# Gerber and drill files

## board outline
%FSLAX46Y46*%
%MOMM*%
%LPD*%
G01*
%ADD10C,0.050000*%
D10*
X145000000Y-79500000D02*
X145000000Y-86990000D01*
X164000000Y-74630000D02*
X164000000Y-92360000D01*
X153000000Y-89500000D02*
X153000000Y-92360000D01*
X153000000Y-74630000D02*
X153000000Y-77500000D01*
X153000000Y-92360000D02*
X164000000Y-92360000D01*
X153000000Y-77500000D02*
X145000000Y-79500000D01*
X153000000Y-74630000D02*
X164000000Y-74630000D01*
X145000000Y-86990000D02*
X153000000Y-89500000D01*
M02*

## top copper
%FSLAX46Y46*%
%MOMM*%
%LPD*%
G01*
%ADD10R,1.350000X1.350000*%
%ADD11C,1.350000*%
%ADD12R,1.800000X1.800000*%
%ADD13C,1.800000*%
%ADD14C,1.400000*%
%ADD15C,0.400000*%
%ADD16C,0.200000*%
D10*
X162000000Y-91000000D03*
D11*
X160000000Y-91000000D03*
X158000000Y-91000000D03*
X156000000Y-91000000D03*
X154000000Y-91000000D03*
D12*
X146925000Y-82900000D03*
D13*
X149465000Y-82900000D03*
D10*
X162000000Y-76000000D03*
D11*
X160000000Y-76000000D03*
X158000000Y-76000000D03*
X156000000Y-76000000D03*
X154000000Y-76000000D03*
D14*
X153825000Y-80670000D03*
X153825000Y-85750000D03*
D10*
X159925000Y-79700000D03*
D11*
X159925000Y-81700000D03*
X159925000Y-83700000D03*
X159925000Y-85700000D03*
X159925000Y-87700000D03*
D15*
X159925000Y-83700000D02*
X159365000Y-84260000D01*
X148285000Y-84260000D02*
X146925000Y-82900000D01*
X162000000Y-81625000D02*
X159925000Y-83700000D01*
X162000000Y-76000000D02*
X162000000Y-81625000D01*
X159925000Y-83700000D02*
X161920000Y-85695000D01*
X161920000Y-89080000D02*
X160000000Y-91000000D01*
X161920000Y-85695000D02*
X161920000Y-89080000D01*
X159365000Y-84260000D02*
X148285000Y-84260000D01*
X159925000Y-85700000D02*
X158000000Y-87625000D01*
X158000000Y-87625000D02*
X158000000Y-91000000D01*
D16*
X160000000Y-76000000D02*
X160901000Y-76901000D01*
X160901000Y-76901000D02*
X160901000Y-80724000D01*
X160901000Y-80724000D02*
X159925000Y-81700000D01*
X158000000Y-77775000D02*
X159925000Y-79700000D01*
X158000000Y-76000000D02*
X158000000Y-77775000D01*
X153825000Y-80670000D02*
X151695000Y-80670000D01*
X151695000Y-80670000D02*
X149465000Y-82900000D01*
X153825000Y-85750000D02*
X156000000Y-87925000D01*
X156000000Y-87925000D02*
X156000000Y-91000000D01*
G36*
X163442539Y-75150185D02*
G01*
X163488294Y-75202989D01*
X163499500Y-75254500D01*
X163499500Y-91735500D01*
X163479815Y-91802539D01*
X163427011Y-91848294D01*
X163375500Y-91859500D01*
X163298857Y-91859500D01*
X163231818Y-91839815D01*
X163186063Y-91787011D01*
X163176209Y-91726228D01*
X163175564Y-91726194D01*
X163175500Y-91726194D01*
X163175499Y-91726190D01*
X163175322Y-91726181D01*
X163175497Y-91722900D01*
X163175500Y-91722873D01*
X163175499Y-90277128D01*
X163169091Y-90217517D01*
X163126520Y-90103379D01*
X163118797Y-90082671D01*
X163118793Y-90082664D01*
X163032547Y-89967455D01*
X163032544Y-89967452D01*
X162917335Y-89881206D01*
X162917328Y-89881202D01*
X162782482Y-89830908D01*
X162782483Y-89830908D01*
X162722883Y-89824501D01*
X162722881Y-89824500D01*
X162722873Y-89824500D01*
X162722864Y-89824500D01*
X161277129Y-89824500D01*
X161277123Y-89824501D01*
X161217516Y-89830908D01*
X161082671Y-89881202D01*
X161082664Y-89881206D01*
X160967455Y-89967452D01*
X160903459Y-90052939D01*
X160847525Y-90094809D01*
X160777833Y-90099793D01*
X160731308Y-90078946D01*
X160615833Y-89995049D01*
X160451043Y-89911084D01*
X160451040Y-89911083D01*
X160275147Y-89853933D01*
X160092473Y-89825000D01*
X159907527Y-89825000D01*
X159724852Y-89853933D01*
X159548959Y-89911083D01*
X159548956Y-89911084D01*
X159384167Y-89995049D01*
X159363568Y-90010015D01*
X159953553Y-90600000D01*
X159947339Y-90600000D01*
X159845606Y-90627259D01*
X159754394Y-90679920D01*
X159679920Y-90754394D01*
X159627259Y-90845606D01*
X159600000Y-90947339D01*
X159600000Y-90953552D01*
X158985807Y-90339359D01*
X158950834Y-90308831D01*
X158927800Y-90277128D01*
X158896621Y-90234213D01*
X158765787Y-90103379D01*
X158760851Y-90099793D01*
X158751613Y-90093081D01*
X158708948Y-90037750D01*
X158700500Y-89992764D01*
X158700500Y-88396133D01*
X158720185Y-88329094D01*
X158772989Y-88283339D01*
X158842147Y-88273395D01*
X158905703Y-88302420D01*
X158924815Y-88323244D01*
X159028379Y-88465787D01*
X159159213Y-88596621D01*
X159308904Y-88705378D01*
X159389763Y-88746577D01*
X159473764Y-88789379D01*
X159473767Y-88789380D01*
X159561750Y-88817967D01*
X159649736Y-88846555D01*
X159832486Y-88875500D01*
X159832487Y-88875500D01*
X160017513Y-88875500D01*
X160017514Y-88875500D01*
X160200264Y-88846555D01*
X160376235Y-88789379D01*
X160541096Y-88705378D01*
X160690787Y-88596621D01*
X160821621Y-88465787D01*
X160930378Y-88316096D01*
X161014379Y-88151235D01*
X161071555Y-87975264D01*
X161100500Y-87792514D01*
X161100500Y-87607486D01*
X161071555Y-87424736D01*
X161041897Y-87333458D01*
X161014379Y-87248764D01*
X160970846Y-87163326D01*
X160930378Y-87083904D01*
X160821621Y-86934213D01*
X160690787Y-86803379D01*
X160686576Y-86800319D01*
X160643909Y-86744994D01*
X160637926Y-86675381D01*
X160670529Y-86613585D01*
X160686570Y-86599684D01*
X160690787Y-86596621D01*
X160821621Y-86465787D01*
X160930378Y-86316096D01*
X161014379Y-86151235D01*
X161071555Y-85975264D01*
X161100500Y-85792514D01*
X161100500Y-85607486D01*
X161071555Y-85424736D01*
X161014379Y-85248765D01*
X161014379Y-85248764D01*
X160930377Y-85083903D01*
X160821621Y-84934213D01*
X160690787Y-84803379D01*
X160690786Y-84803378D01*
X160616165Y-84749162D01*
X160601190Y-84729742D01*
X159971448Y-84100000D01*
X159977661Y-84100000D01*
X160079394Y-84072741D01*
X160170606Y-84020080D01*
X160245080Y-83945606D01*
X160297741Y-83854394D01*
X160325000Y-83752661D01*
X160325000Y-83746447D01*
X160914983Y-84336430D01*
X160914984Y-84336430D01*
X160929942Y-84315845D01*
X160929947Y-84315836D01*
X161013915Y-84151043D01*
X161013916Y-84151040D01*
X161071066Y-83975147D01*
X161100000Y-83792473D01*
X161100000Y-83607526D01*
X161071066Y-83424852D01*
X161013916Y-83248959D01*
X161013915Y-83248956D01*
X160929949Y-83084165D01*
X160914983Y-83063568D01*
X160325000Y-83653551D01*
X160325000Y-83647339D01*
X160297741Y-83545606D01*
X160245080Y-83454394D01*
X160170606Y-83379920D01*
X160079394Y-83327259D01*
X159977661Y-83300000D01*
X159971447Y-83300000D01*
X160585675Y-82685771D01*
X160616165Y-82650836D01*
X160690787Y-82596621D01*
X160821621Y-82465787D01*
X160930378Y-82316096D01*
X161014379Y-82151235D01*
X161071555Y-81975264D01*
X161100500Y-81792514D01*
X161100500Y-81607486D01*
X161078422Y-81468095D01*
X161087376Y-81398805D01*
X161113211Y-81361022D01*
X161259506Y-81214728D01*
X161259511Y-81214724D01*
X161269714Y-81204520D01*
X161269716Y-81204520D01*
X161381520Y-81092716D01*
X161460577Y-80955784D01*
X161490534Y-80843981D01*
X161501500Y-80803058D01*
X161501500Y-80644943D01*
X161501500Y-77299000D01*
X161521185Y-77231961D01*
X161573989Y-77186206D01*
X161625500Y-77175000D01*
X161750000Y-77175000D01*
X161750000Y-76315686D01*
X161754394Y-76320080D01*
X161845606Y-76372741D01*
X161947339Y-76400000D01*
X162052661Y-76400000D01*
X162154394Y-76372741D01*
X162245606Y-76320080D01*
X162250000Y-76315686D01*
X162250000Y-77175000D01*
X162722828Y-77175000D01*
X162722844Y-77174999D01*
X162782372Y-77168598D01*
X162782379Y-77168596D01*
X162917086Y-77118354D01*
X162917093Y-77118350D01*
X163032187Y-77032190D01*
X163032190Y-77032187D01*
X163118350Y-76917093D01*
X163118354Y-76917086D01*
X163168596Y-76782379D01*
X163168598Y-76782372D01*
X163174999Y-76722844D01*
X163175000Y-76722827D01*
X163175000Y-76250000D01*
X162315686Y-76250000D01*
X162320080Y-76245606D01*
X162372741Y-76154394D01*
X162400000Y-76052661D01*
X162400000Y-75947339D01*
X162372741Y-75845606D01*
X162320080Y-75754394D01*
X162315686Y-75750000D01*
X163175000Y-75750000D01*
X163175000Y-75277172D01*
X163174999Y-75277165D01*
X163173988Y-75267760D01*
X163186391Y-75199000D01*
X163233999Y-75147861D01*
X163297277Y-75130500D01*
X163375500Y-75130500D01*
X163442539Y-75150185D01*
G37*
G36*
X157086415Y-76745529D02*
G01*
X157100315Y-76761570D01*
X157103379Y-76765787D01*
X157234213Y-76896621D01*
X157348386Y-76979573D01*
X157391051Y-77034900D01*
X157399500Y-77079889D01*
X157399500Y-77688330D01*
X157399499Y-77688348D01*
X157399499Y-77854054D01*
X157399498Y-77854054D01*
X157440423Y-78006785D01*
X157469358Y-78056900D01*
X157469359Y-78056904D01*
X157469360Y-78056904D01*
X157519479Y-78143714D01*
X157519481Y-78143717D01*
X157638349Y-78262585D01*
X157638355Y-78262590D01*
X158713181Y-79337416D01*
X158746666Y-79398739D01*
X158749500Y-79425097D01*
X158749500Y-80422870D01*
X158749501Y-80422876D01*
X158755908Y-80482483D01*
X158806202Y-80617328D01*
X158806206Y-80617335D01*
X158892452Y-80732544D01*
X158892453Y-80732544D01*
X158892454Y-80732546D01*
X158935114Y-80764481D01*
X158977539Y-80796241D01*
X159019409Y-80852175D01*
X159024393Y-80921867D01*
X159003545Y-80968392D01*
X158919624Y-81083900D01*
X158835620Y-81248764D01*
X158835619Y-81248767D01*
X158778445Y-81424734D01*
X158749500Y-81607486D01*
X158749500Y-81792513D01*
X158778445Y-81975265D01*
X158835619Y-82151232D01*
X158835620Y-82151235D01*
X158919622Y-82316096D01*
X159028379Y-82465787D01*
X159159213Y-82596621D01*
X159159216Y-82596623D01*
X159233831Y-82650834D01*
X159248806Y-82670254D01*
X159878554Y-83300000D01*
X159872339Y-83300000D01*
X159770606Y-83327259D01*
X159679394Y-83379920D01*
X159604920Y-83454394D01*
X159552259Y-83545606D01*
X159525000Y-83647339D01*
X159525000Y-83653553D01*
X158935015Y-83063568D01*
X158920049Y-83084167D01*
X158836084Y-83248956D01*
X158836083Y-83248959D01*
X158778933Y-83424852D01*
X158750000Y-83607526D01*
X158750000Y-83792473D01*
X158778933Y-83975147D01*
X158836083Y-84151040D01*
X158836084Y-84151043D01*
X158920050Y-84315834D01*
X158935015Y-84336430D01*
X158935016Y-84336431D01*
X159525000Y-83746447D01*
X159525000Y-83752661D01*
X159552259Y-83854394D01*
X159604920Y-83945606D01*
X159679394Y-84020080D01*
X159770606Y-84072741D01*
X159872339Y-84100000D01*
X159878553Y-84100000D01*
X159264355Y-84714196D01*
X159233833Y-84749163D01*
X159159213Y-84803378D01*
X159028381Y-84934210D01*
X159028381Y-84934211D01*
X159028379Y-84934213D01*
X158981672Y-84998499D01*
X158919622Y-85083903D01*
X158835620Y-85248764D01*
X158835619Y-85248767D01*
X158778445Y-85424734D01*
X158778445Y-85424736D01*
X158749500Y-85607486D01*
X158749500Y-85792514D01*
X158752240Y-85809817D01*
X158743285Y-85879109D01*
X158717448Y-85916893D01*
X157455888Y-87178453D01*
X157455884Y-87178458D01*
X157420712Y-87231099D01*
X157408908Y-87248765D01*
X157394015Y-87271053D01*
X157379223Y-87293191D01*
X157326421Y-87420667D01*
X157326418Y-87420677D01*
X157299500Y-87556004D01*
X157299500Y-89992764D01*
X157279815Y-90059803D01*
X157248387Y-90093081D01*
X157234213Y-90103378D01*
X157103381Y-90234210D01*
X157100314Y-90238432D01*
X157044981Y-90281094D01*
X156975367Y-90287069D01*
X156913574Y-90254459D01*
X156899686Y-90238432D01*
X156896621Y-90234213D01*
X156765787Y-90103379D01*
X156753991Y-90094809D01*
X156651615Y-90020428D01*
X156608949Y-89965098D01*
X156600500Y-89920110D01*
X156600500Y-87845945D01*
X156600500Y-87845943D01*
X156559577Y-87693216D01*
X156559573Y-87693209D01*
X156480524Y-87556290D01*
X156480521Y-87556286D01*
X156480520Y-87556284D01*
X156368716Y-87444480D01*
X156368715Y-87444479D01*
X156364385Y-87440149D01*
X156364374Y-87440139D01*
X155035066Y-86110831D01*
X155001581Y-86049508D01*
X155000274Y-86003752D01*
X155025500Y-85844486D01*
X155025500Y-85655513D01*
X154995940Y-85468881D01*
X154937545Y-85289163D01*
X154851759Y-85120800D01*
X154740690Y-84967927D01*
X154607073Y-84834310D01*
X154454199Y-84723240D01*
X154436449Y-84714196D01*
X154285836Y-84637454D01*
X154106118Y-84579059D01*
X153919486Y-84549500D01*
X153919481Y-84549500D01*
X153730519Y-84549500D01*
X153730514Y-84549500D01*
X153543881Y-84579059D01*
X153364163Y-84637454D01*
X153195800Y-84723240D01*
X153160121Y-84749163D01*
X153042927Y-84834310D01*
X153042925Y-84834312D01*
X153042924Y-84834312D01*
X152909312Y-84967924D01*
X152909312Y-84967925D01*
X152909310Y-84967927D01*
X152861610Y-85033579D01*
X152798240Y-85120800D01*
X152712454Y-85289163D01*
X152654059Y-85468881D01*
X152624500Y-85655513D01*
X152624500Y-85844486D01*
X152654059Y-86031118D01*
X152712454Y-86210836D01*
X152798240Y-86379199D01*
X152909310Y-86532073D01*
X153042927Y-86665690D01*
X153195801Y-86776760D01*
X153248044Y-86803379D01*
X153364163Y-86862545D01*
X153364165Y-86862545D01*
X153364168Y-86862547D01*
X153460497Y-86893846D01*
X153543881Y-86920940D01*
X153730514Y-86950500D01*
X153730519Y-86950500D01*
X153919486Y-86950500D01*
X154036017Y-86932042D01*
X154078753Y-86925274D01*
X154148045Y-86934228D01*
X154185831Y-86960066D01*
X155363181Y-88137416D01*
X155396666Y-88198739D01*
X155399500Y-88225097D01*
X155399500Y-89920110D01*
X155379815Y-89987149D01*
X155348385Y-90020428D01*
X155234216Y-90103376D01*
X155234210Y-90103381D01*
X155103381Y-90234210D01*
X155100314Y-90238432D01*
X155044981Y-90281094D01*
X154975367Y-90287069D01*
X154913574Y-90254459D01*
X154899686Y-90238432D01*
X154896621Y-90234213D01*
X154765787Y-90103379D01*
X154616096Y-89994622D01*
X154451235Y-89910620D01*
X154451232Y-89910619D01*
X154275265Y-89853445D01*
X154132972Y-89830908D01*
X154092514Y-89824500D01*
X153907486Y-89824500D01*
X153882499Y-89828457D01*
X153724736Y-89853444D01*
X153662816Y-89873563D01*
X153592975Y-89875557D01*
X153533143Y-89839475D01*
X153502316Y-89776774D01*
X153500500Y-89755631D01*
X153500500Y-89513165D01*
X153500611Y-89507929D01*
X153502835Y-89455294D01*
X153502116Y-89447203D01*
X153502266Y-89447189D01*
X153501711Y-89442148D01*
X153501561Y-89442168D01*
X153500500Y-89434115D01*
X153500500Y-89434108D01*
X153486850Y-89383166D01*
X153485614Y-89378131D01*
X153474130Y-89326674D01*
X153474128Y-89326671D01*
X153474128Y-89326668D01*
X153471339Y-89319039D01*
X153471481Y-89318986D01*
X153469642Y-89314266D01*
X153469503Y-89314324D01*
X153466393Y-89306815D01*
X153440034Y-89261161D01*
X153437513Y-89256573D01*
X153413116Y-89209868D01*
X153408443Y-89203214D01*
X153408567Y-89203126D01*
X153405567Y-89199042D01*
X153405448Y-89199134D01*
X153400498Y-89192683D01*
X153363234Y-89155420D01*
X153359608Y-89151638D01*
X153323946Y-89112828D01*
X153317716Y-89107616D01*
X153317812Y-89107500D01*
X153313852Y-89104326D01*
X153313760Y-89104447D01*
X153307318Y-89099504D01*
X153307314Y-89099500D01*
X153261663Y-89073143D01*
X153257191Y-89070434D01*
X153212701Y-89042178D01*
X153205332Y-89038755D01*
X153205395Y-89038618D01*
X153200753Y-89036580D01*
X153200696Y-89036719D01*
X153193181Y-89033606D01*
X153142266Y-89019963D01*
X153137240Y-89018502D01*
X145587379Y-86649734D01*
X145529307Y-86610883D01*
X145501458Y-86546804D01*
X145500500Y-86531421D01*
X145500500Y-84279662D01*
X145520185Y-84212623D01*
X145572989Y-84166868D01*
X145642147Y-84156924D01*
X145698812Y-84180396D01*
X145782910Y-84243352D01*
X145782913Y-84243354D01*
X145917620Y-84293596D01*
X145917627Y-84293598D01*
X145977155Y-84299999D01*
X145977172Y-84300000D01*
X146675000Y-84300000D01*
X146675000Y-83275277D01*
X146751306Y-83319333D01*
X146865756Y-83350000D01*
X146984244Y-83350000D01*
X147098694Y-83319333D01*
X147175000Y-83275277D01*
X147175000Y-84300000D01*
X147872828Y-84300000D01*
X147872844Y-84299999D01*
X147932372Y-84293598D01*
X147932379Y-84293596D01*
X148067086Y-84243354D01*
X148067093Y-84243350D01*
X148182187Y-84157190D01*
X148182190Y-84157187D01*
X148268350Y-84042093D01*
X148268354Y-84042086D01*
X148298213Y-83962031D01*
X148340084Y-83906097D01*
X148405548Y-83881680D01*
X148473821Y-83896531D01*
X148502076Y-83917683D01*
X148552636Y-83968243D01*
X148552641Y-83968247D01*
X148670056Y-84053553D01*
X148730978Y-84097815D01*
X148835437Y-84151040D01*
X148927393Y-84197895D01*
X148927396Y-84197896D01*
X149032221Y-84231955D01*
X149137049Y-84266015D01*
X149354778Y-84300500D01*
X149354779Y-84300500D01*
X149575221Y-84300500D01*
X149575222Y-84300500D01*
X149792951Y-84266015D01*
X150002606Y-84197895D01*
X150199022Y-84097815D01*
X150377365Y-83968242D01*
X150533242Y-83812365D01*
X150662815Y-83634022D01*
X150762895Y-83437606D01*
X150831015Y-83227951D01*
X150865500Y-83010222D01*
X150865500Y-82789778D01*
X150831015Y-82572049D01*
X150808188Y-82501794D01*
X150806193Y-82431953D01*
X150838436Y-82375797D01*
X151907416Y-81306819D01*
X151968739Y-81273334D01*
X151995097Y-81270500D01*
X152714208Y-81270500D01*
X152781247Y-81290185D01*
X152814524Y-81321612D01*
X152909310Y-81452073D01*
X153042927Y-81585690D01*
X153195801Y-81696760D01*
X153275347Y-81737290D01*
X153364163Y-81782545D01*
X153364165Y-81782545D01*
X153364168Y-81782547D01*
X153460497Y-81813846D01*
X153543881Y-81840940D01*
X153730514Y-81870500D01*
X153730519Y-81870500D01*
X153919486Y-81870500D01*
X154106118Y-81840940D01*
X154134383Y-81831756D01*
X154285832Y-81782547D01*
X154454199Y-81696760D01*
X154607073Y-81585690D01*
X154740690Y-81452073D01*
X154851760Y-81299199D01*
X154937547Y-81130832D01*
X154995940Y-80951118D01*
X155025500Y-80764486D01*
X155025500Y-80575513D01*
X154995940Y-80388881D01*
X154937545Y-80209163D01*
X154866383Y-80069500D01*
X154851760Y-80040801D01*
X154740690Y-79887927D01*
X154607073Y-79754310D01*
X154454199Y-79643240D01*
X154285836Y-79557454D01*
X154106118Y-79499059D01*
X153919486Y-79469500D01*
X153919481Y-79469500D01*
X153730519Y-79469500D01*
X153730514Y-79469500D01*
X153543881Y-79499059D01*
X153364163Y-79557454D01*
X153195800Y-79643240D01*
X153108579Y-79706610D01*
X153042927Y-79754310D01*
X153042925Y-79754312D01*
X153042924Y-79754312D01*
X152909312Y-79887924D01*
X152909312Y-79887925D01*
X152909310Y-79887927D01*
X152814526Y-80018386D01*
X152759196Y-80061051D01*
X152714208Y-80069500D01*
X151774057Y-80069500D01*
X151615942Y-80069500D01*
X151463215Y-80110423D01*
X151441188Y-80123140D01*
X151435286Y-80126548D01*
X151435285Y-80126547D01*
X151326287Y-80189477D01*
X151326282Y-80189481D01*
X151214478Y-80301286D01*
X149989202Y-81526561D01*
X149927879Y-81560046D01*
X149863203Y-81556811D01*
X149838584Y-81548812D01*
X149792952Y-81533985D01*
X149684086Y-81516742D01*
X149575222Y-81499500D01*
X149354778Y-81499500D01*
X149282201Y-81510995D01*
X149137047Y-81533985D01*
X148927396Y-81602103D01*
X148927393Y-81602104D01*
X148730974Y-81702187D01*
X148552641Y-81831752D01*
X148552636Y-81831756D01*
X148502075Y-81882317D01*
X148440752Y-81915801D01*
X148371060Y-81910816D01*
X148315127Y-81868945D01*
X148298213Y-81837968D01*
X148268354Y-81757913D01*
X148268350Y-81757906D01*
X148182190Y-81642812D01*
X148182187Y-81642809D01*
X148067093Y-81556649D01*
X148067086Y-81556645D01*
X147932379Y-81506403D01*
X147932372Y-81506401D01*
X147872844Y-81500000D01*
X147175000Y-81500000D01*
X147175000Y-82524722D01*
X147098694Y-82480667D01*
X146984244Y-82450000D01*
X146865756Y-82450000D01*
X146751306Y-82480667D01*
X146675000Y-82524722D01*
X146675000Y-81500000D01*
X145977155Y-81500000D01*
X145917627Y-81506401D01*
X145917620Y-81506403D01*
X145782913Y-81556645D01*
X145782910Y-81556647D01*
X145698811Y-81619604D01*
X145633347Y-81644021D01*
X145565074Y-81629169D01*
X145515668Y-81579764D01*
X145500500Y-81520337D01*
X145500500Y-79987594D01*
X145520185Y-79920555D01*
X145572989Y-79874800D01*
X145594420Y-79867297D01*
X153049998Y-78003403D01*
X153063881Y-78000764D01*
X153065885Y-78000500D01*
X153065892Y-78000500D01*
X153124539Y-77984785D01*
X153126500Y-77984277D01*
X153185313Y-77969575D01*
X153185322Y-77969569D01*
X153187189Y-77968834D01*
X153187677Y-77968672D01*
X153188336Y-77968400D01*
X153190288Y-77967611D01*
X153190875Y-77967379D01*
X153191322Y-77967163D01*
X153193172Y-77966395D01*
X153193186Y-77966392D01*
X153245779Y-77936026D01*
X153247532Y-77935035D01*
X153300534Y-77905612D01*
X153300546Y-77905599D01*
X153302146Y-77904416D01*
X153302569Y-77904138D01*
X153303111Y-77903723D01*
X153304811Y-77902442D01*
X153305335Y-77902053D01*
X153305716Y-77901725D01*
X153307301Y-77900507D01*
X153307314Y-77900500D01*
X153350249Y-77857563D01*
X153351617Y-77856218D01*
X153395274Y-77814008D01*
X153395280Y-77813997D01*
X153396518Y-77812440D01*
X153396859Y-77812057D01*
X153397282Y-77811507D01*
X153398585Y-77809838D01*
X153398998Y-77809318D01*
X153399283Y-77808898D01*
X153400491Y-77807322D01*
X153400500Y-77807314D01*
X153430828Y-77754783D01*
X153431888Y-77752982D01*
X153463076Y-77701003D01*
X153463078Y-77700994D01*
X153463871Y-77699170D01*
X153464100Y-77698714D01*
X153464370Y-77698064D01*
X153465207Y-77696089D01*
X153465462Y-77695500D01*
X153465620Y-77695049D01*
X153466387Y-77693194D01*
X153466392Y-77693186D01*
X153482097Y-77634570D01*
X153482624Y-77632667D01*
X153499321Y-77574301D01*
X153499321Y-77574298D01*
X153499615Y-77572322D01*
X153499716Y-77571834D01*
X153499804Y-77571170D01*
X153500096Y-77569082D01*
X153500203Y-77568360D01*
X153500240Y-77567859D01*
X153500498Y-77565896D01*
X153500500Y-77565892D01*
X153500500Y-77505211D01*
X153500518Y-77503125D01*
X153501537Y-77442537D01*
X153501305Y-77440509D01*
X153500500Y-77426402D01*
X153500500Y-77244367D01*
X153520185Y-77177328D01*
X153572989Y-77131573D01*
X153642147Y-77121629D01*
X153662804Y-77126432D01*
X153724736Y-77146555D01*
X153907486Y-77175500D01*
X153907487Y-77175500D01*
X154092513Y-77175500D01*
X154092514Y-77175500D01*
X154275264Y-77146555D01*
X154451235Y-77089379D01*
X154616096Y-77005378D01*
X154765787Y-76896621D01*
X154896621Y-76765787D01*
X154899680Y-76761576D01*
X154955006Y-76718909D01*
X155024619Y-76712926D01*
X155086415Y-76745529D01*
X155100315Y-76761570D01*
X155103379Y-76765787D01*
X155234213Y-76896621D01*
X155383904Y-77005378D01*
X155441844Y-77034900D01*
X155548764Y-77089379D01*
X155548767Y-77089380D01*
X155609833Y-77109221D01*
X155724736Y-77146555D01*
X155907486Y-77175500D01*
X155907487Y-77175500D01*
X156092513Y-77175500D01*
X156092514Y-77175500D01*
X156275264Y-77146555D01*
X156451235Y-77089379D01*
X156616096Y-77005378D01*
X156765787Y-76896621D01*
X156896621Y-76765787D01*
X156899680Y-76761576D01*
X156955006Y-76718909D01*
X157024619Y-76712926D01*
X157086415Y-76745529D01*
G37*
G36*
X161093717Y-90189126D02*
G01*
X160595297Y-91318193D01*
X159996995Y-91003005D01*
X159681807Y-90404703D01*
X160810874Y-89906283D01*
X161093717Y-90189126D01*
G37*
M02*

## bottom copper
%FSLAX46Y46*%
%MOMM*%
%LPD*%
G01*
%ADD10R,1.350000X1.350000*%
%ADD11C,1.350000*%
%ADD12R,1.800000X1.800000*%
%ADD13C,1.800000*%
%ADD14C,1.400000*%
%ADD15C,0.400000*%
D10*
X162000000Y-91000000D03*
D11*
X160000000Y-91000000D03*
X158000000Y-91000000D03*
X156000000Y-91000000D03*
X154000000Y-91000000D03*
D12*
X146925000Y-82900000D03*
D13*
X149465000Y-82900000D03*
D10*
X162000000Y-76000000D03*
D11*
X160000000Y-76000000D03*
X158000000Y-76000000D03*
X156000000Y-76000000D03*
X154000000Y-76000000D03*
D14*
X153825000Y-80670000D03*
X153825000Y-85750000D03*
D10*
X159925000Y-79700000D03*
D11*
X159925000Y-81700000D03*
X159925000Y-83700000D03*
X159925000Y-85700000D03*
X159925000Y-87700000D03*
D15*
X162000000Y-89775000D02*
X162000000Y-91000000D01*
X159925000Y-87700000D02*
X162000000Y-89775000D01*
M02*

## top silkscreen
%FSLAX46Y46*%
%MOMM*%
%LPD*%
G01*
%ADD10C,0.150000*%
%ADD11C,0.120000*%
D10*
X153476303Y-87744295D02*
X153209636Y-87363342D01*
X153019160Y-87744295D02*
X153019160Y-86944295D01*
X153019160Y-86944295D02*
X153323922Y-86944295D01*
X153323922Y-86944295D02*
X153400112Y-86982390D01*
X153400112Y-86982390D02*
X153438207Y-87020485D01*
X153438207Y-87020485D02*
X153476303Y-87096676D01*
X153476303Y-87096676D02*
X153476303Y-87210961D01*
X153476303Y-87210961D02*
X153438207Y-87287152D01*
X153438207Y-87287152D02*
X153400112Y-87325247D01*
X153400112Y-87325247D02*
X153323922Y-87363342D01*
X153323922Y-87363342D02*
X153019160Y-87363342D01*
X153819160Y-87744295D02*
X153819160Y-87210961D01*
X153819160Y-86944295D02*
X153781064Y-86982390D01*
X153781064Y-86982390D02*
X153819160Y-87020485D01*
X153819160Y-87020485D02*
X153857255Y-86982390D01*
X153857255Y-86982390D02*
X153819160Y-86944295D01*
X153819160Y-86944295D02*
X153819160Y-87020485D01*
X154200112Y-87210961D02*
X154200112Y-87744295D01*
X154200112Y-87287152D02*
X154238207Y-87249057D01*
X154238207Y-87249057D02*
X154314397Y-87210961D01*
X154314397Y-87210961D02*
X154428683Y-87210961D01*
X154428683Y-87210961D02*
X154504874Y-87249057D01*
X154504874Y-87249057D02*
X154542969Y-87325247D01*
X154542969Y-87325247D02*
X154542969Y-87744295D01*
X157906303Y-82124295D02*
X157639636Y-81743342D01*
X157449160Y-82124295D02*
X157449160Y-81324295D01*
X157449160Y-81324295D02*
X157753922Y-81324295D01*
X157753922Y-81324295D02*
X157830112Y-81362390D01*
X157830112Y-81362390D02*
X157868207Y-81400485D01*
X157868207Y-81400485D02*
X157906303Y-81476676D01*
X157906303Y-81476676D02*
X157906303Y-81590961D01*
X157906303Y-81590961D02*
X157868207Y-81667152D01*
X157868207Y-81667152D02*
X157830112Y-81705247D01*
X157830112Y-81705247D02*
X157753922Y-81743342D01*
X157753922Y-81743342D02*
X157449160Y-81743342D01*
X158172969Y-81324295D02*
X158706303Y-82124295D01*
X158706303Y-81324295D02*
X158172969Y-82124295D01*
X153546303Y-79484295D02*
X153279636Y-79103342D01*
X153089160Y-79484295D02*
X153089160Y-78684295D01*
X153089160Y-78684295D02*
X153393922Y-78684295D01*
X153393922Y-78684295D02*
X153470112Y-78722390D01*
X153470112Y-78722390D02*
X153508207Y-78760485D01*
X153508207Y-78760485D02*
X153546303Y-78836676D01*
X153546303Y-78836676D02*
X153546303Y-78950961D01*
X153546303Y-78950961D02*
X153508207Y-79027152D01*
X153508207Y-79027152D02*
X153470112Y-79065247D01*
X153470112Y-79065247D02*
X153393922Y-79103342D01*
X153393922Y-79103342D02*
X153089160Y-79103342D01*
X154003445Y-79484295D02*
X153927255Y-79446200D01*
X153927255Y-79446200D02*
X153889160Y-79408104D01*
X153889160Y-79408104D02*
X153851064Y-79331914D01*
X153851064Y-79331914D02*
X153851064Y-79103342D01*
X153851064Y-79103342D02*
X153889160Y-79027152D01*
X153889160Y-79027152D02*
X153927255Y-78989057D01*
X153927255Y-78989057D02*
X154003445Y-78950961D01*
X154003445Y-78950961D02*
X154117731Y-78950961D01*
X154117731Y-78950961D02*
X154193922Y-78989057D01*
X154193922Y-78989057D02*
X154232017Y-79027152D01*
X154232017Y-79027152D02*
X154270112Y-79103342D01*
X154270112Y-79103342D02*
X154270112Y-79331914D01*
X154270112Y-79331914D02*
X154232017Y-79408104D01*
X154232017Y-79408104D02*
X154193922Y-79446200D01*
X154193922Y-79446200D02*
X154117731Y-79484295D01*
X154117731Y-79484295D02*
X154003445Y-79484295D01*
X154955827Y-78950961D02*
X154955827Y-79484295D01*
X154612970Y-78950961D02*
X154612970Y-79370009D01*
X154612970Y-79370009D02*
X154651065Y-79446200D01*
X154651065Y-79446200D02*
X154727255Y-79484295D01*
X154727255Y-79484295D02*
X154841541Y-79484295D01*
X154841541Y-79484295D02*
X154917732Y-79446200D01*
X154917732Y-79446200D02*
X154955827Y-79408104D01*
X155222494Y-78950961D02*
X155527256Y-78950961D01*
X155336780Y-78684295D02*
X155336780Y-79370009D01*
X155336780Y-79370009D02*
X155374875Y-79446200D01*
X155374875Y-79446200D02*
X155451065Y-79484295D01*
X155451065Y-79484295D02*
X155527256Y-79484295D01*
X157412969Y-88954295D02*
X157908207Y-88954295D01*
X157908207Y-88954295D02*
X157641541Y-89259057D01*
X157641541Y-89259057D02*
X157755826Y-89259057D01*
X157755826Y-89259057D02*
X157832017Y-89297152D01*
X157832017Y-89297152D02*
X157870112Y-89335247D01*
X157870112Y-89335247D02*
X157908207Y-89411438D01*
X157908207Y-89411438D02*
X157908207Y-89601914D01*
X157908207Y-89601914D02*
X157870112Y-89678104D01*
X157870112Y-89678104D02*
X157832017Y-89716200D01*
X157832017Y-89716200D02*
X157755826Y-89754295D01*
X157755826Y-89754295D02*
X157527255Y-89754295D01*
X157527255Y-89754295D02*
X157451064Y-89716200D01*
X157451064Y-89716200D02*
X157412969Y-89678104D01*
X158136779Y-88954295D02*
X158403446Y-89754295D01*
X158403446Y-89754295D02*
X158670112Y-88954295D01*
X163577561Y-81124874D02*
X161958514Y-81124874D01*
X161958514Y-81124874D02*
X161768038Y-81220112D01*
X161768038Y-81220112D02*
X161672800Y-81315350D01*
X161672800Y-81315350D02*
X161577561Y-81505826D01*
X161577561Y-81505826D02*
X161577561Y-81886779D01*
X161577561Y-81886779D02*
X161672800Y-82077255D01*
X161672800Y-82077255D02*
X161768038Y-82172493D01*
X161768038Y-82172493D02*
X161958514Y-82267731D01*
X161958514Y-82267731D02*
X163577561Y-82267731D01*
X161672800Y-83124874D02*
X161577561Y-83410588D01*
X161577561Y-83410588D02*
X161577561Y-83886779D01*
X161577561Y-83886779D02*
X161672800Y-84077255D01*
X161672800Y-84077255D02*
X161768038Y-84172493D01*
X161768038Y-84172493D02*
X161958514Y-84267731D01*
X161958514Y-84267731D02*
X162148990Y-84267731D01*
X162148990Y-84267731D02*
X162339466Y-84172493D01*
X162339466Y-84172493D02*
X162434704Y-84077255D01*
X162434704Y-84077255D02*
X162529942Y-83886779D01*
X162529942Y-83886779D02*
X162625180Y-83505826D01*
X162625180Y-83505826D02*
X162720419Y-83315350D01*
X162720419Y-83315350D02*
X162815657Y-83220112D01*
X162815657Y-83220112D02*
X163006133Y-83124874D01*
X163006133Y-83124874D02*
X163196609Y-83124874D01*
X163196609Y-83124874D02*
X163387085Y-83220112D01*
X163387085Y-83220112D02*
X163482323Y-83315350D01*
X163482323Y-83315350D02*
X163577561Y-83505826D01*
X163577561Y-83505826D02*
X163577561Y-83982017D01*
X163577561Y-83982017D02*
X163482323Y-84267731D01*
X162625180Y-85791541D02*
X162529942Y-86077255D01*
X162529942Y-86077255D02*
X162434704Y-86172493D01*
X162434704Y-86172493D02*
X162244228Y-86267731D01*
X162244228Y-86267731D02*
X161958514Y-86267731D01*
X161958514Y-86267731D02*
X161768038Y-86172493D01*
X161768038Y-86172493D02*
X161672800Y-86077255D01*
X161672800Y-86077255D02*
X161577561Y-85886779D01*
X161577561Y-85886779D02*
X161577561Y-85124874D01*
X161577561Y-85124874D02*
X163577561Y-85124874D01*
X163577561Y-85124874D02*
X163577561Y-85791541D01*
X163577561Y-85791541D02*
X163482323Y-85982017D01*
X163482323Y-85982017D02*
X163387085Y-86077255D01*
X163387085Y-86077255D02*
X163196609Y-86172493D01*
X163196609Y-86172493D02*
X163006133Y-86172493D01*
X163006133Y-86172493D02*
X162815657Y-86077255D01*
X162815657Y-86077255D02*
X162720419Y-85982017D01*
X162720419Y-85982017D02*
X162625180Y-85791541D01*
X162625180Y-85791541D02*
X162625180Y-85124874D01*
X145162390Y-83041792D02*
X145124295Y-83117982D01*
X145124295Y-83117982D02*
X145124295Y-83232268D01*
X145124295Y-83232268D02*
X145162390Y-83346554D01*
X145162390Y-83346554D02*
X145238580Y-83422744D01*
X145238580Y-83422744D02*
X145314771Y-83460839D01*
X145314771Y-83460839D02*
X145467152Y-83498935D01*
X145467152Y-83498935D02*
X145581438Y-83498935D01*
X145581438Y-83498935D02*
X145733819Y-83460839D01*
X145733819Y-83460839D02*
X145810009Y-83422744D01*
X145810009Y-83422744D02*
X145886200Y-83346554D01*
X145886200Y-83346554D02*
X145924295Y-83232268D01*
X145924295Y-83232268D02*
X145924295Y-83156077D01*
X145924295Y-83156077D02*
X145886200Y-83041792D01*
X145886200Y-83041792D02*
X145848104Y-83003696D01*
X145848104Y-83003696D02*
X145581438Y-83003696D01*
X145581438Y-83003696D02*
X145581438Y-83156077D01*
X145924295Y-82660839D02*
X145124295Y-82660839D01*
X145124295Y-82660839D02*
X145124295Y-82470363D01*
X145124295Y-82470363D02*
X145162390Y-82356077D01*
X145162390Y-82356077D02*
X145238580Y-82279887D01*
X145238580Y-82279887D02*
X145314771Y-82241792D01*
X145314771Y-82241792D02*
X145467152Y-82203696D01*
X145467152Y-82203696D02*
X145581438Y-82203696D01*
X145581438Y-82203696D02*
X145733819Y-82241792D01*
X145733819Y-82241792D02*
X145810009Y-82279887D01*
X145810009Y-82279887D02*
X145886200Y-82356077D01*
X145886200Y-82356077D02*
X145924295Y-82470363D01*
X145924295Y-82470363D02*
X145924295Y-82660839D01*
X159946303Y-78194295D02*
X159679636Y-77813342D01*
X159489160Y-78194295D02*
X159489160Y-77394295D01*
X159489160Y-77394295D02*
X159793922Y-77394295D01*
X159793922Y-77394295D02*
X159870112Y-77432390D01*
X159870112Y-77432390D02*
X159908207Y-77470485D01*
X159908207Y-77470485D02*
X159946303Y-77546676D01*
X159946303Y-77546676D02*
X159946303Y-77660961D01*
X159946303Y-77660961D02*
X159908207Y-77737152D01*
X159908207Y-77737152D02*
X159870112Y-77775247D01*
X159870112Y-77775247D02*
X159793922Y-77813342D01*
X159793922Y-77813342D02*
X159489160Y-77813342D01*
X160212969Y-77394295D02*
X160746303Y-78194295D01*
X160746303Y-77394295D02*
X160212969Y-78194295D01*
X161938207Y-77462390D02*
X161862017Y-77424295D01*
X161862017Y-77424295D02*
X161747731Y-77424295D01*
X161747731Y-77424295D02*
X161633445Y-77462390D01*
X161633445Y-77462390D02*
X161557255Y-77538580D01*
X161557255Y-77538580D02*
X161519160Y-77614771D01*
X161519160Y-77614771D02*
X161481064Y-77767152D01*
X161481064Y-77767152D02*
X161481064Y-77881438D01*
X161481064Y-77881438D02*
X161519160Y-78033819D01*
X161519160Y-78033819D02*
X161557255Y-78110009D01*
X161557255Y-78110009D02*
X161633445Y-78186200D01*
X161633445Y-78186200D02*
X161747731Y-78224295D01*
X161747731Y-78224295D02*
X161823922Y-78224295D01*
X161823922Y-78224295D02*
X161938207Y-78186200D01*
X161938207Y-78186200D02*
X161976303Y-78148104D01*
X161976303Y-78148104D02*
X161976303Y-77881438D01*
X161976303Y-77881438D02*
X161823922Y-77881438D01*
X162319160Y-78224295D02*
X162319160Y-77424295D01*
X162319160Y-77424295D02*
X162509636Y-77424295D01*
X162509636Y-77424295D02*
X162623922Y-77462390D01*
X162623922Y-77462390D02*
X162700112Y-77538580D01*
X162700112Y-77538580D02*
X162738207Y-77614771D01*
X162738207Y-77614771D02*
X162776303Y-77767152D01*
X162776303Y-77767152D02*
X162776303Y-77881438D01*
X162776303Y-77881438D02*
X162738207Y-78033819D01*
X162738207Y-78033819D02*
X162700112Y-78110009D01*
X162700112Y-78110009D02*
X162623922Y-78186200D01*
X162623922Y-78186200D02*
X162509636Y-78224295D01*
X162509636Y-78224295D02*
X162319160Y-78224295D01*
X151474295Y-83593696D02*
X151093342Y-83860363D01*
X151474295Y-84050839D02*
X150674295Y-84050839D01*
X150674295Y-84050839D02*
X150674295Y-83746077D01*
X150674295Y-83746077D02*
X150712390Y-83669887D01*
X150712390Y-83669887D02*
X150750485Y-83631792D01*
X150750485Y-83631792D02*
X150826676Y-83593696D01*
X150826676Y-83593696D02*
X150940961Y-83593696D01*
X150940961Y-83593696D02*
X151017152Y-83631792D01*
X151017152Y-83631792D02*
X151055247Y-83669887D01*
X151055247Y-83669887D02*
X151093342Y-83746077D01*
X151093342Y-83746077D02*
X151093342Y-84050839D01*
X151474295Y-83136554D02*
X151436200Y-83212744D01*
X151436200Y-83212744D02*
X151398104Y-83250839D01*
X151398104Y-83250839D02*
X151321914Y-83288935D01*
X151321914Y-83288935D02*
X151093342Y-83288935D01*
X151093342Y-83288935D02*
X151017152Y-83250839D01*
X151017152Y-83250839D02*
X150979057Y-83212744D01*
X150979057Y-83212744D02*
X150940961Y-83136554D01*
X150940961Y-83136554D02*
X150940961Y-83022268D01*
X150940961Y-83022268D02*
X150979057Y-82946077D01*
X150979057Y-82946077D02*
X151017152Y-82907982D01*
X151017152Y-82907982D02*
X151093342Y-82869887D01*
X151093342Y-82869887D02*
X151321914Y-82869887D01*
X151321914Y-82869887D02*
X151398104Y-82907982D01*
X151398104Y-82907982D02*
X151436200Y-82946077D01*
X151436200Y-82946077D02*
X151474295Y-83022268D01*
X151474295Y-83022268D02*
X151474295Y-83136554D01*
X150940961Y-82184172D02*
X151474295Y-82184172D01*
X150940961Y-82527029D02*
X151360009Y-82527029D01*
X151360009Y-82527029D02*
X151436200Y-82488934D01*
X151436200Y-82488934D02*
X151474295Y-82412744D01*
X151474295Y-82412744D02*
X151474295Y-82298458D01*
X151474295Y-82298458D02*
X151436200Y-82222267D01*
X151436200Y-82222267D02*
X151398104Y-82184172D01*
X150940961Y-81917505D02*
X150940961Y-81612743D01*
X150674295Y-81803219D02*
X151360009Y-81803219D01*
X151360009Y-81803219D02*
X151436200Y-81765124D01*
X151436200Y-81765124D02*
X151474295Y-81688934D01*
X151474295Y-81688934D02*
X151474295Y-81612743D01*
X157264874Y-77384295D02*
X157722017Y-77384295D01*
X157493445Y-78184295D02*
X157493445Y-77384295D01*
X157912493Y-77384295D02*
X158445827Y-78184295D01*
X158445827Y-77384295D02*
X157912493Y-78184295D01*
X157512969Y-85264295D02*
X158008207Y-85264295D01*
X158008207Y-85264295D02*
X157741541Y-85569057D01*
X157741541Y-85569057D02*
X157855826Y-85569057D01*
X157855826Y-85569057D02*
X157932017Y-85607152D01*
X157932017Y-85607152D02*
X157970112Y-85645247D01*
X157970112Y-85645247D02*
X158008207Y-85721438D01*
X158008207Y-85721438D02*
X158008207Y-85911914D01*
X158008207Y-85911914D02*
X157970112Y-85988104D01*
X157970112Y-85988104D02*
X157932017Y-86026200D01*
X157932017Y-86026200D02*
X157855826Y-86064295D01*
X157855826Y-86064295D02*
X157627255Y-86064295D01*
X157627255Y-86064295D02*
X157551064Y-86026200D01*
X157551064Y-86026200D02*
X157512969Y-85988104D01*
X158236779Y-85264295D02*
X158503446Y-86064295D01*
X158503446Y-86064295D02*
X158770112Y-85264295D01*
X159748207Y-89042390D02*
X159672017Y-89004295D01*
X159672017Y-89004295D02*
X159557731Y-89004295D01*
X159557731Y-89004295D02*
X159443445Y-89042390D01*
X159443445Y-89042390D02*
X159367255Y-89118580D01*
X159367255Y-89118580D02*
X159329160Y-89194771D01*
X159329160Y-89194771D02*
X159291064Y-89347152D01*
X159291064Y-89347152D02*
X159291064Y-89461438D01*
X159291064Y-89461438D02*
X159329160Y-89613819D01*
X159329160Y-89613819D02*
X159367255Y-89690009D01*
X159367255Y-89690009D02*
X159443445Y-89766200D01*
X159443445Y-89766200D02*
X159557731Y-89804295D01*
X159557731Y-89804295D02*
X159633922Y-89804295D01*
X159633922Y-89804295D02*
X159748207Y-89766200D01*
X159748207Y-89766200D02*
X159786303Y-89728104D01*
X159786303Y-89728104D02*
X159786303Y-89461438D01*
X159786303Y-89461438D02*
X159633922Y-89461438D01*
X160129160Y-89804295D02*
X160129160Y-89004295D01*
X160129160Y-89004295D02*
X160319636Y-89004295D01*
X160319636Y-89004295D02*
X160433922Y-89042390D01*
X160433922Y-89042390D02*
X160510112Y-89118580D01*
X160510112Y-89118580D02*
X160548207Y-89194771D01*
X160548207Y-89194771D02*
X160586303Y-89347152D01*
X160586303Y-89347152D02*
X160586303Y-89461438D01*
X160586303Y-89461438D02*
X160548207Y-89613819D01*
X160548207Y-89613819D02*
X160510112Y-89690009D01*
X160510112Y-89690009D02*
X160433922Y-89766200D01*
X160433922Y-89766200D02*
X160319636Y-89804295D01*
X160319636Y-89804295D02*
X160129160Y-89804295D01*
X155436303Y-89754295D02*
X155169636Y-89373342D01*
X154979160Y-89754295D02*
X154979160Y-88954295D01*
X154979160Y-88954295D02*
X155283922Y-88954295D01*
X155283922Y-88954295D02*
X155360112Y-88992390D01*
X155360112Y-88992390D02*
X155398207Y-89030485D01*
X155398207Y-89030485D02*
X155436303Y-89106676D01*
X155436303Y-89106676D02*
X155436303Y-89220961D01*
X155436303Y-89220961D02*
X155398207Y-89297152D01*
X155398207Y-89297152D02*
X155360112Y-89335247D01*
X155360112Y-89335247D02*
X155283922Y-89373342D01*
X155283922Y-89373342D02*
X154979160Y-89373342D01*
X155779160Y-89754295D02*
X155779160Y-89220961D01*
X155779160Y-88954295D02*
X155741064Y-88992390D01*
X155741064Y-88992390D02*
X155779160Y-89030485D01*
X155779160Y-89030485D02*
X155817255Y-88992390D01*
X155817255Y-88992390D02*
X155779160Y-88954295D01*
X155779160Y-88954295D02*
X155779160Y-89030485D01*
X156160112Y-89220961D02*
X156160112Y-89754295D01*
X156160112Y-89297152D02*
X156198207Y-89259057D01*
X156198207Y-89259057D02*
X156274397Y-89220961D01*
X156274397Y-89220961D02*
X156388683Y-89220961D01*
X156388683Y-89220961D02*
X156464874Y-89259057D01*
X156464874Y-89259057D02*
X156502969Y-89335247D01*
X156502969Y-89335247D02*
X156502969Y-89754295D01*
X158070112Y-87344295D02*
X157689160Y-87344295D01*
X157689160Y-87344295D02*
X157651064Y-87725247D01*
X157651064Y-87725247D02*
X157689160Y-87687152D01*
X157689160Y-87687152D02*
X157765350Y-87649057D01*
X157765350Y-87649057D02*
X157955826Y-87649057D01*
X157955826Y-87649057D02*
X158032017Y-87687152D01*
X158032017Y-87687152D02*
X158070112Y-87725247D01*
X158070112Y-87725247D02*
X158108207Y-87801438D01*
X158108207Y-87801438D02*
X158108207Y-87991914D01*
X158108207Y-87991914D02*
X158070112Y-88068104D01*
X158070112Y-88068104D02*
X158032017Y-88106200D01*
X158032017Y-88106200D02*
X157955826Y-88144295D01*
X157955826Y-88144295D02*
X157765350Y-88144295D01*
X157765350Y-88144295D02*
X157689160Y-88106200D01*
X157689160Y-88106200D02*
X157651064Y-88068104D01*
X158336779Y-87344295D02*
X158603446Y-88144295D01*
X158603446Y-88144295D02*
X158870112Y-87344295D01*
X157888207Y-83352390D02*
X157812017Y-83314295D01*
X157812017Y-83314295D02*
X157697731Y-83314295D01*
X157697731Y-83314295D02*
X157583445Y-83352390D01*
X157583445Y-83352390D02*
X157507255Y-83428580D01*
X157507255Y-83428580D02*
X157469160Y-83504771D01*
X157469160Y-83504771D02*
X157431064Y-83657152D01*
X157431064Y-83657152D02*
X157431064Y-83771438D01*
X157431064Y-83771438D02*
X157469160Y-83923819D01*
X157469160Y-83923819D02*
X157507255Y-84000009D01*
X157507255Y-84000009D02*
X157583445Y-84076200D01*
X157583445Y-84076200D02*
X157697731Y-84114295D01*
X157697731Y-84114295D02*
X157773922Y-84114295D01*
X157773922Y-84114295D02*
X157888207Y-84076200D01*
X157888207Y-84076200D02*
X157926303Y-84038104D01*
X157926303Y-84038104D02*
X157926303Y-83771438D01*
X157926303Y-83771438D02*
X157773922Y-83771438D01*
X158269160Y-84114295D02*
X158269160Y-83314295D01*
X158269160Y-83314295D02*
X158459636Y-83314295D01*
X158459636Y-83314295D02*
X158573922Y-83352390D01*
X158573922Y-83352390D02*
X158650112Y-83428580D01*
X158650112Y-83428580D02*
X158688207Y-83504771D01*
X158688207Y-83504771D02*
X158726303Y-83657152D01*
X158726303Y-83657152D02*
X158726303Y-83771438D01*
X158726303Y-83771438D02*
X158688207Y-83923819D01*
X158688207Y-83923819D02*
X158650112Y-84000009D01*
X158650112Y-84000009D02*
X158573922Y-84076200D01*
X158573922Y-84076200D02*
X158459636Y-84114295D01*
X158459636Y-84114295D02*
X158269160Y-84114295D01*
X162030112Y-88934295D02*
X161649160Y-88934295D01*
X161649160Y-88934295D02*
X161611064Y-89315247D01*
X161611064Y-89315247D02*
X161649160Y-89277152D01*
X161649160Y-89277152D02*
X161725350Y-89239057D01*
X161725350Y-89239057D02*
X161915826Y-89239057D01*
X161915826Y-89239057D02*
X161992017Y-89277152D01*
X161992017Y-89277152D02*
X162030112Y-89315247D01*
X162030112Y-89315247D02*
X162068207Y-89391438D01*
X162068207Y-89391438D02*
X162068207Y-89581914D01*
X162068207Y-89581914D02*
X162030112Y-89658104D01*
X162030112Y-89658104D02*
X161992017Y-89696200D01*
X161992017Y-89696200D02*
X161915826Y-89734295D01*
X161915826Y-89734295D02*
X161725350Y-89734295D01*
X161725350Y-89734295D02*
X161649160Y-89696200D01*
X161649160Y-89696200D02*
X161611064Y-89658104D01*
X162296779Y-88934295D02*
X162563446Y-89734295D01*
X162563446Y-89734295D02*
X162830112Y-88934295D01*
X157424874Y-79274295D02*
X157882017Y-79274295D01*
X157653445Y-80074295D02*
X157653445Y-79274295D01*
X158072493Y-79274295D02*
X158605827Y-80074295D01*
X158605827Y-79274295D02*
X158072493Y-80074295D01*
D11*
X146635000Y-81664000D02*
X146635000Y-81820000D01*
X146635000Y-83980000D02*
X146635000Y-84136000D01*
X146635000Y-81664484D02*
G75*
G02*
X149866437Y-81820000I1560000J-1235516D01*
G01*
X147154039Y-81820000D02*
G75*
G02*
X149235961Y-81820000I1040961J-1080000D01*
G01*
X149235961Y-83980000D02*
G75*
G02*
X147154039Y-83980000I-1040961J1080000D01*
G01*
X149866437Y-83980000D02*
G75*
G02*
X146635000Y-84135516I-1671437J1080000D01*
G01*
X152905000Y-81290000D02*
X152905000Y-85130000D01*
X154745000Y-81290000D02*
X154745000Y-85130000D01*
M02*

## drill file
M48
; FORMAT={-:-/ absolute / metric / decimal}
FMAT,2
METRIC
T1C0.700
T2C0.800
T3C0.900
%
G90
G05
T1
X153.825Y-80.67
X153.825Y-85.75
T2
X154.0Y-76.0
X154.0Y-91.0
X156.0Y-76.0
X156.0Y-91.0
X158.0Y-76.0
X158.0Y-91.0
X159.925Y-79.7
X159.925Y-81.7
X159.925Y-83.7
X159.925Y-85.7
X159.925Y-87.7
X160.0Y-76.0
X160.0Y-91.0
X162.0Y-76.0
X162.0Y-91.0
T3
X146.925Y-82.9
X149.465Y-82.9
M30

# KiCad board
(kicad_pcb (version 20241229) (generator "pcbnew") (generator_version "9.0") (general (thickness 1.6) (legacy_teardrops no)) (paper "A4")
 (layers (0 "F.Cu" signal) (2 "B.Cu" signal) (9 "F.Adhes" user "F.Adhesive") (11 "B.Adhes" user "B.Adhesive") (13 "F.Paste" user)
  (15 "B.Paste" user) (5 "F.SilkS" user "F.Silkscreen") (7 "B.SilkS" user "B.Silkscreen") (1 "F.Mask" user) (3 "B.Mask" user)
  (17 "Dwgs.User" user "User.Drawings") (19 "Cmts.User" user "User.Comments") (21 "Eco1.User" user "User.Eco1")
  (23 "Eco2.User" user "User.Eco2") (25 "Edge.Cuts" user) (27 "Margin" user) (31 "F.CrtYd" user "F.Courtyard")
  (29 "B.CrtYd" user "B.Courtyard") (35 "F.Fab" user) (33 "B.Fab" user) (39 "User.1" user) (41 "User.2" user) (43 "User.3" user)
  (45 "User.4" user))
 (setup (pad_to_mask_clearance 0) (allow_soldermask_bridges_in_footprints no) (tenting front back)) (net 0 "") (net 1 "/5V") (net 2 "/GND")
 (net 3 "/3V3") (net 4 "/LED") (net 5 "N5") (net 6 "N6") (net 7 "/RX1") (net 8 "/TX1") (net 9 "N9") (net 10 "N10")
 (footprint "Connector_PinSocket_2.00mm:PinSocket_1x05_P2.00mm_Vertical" (layer "F.Cu") (at 162 91 -90)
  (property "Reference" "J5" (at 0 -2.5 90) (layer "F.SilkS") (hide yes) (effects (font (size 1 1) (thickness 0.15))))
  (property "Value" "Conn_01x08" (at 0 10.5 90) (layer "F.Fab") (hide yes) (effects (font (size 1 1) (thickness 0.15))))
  (pad "1" thru_hole rect (at 0 0 270) (size 1.35 1.35) (drill 0.8) (layers "*.Cu" "*.Mask") (remove_unused_layers no) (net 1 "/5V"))
  (pad "2" thru_hole circle (at 0 2 270) (size 1.35 1.35) (drill 0.8) (layers "*.Cu" "*.Mask") (remove_unused_layers no) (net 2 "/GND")
   (teardrops (best_length_ratio 0.5) (max_length 1) (best_width_ratio 1) (max_width 2) (curved_edges no) (filter_ratio 0.9) (enabled yes)
    (allow_two_segments yes) (prefer_zone_connections yes)))
  (pad "3" thru_hole circle (at 0 4 270) (size 1.35 1.35) (drill 0.8) (layers "*.Cu" "*.Mask") (remove_unused_layers no) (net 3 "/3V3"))
  (pad "4" thru_hole circle (at 0 6 270) (size 1.35 1.35) (drill 0.8) (layers "*.Cu" "*.Mask") (remove_unused_layers no) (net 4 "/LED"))
  (pad "5" thru_hole circle (at 0 8 270) (size 1.35 1.35) (drill 0.8) (layers "*.Cu" "*.Mask") (remove_unused_layers no) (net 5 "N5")))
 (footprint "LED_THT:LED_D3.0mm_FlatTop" (layer "F.Cu") (at 146.925 82.9)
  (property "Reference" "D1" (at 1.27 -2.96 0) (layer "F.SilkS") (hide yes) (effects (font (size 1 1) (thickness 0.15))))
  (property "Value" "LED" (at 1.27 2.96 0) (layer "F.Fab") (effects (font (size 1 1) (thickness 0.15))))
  (fp_line (start -0.29 -1.236) (end -0.29 -1.08) (stroke (width 0.12) (type solid)) (layer "F.SilkS"))
  (fp_line (start -0.29 1.08) (end -0.29 1.236) (stroke (width 0.12) (type solid)) (layer "F.SilkS"))
  (fp_arc (start -0.29 -1.235516) (mid 1.36566 -1.987699) (end 2.941437 -1.08) (stroke (width 0.12) (type solid)) (layer "F.SilkS"))
  (fp_arc (start 0.229039 -1.08) (mid 1.27 -1.5) (end 2.310961 -1.08) (stroke (width 0.12) (type solid)) (layer "F.SilkS"))
  (fp_arc (start 2.310961 1.08) (mid 1.27 1.5) (end 0.229039 1.08) (stroke (width 0.12) (type solid)) (layer "F.SilkS"))
  (fp_arc (start 2.941437 1.08) (mid 1.36566 1.987699) (end -0.29 1.235516) (stroke (width 0.12) (type solid)) (layer "F.SilkS"))
  (pad "1" thru_hole rect (at 0 0) (size 1.8 1.8) (drill 0.9) (layers "*.Cu" "*.Mask") (remove_unused_layers no) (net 2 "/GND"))
  (pad "2" thru_hole circle (at 2.54 0) (size 1.8 1.8) (drill 0.9) (layers "*.Cu" "*.Mask") (remove_unused_layers no) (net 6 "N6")))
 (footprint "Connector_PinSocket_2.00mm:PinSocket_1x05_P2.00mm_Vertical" (layer "F.Cu") (at 162 76 -90)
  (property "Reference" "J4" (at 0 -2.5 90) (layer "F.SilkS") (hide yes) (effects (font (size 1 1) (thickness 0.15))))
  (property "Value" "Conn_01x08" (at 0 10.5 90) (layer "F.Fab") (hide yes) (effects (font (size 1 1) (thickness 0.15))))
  (pad "1" thru_hole rect (at 0 0 270) (size 1.35 1.35) (drill 0.8) (layers "*.Cu" "*.Mask") (remove_unused_layers no) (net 2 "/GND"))
  (pad "2" thru_hole circle (at 0 2 270) (size 1.35 1.35) (drill 0.8) (layers "*.Cu" "*.Mask") (remove_unused_layers no) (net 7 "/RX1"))
  (pad "3" thru_hole circle (at 0 4 270) (size 1.35 1.35) (drill 0.8) (layers "*.Cu" "*.Mask") (remove_unused_layers no) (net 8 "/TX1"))
  (pad "4" thru_hole circle (at 0 6 270) (size 1.35 1.35) (drill 0.8) (layers "*.Cu" "*.Mask") (remove_unused_layers no) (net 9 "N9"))
  (pad "5" thru_hole circle (at 0 8 270) (size 1.35 1.35) (drill 0.8) (layers "*.Cu" "*.Mask") (remove_unused_layers no) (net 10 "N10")))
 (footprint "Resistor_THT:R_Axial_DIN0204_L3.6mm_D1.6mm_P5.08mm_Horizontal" (layer "F.Cu") (at 153.825 80.67 -90)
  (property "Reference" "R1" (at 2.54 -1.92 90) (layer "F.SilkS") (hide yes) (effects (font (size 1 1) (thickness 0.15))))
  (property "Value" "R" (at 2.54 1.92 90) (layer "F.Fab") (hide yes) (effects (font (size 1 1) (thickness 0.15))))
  (fp_line (start 0.62 0.92) (end 4.46 0.92) (stroke (width 0.12) (type solid)) (layer "F.SilkS"))
  (fp_line (start 0.62 -0.92) (end 4.46 -0.92) (stroke (width 0.12) (type solid)) (layer "F.SilkS"))
  (pad "1" thru_hole circle (at 0 0 270) (size 1.4 1.4) (drill 0.7) (layers "*.Cu" "*.Mask") (remove_unused_layers no) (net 6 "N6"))
  (pad "2" thru_hole circle (at 5.08 0 270) (size 1.4 1.4) (drill 0.7) (layers "*.Cu" "*.Mask") (remove_unused_layers no) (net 4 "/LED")))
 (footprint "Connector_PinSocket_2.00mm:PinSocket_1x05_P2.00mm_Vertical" (layer "F.Cu") (at 159.925 79.7)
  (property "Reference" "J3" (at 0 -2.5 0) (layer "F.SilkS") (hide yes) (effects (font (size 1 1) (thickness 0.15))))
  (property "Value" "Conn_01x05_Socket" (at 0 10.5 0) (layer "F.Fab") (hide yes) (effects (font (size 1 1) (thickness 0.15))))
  (pad "1" thru_hole rect (at 0 0) (size 1.35 1.35) (drill 0.8) (layers "*.Cu" "*.Mask") (remove_unused_layers no) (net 8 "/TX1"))
  (pad "2" thru_hole circle (at 0 2) (size 1.35 1.35) (drill 0.8) (layers "*.Cu" "*.Mask") (remove_unused_layers no) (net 7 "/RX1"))
  (pad "3" thru_hole circle (at 0 4) (size 1.35 1.35) (drill 0.8) (layers "*.Cu" "*.Mask") (remove_unused_layers no) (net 2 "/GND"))
  (pad "4" thru_hole circle (at 0 6) (size 1.35 1.35) (drill 0.8) (layers "*.Cu" "*.Mask") (remove_unused_layers no) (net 3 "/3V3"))
  (pad "5" thru_hole circle (at 0 8) (size 1.35 1.35) (drill 0.8) (layers "*.Cu" "*.Mask") (remove_unused_layers no) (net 1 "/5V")))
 (gr_line (start 145 79.5) (end 145 86.99) (stroke (width 0.05) (type solid)) (layer "Edge.Cuts"))
 (gr_line (start 164 74.63) (end 164 92.36) (stroke (width 0.05) (type default)) (layer "Edge.Cuts"))
 (gr_line (start 153 89.5) (end 153 92.36) (stroke (width 0.05) (type solid)) (layer "Edge.Cuts"))
 (gr_line (start 153 74.63) (end 153 77.5) (stroke (width 0.05) (type solid)) (layer "Edge.Cuts"))
 (gr_line (start 153 92.36) (end 164 92.36) (stroke (width 0.05) (type solid)) (layer "Edge.Cuts"))
 (gr_line (start 153 77.5) (end 145 79.5) (stroke (width 0.05) (type default)) (layer "Edge.Cuts"))
 (gr_line (start 153 74.63) (end 164 74.63) (stroke (width 0.05) (type solid)) (layer "Edge.Cuts"))
 (gr_line (start 145 86.99) (end 153 89.5) (stroke (width 0.05) (type default)) (layer "Edge.Cuts"))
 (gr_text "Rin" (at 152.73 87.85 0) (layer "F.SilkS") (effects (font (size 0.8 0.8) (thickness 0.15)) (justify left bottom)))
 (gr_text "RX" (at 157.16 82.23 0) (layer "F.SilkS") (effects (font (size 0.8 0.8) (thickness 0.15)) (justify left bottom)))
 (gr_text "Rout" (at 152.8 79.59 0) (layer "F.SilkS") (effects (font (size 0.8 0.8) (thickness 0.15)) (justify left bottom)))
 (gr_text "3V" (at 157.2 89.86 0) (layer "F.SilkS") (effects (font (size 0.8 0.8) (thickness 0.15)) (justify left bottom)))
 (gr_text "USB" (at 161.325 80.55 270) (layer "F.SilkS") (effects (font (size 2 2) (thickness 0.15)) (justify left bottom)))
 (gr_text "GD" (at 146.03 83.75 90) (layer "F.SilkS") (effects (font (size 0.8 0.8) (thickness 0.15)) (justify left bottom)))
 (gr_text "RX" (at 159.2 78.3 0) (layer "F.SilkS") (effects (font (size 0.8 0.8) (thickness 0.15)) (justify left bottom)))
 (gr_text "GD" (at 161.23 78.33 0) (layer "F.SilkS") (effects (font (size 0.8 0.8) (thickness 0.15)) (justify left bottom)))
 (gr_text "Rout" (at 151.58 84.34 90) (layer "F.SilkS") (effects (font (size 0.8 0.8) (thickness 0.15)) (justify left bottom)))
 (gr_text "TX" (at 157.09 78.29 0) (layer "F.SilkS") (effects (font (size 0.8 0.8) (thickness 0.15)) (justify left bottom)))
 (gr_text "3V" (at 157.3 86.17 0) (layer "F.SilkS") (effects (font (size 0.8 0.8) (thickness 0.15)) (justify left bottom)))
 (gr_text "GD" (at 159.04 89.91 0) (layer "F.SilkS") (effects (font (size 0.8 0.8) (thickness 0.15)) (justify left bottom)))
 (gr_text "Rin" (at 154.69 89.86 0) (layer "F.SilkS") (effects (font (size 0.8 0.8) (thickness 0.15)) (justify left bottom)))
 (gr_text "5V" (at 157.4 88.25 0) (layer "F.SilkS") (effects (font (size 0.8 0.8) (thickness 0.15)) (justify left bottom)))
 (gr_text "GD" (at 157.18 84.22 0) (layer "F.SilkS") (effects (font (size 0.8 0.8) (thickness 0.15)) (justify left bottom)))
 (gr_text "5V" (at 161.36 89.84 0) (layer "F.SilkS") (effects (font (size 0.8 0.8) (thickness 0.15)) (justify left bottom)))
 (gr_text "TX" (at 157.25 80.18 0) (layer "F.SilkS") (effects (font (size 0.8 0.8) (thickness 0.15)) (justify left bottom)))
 (segment (start 159.925 83.7) (end 159.365 84.26) (width 0.4) (layer "F.Cu") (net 2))
 (segment (start 148.285 84.26) (end 146.925 82.9) (width 0.4) (layer "F.Cu") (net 2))
 (segment (start 162 81.625) (end 159.925 83.7) (width 0.4) (layer "F.Cu") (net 2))
 (segment (start 162 76) (end 162 81.625) (width 0.4) (layer "F.Cu") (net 2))
 (segment (start 159.925 83.7) (end 161.92 85.695) (width 0.4) (layer "F.Cu") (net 2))
 (segment (start 161.92 89.08) (end 160 91) (width 0.4) (layer "F.Cu") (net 2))
 (segment (start 161.92 85.695) (end 161.92 89.08) (width 0.4) (layer "F.Cu") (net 2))
 (segment (start 159.365 84.26) (end 148.285 84.26) (width 0.4) (layer "F.Cu") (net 2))
 (segment (start 159.925 85.7) (end 158 87.625) (width 0.4) (layer "F.Cu") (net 3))
 (segment (start 158 87.625) (end 158 91) (width 0.4) (layer "F.Cu") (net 3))
 (segment (start 160 76) (end 160.901 76.901) (width 0.2) (layer "F.Cu") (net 7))
 (segment (start 160.901 76.901) (end 160.901 80.724) (width 0.2) (layer "F.Cu") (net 7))
 (segment (start 160.901 80.724) (end 159.925 81.7) (width 0.2) (layer "F.Cu") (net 7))
 (segment (start 158 77.775) (end 159.925 79.7) (width 0.2) (layer "F.Cu") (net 8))
 (segment (start 158 76) (end 158 77.775) (width 0.2) (layer "F.Cu") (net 8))
 (segment (start 162 89.775) (end 162 91) (width 0.4) (layer "B.Cu") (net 1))
 (segment (start 159.925 87.7) (end 162 89.775) (width 0.4) (layer "B.Cu") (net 1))
 (segment (start 153.825 80.67) (end 151.695 80.67) (width 0.2) (layer "F.Cu") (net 6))
 (segment (start 151.695 80.67) (end 149.465 82.9) (width 0.2) (layer "F.Cu") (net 6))
 (segment (start 153.825 85.75) (end 156 87.925) (width 0.2) (layer "F.Cu") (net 4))
 (segment (start 156 87.925) (end 156 91) (width 0.2) (layer "F.Cu") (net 4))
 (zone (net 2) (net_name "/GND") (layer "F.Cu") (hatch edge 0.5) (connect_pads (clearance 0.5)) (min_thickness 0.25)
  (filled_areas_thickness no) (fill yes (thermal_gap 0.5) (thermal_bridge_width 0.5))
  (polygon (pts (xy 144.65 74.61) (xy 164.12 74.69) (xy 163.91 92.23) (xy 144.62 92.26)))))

